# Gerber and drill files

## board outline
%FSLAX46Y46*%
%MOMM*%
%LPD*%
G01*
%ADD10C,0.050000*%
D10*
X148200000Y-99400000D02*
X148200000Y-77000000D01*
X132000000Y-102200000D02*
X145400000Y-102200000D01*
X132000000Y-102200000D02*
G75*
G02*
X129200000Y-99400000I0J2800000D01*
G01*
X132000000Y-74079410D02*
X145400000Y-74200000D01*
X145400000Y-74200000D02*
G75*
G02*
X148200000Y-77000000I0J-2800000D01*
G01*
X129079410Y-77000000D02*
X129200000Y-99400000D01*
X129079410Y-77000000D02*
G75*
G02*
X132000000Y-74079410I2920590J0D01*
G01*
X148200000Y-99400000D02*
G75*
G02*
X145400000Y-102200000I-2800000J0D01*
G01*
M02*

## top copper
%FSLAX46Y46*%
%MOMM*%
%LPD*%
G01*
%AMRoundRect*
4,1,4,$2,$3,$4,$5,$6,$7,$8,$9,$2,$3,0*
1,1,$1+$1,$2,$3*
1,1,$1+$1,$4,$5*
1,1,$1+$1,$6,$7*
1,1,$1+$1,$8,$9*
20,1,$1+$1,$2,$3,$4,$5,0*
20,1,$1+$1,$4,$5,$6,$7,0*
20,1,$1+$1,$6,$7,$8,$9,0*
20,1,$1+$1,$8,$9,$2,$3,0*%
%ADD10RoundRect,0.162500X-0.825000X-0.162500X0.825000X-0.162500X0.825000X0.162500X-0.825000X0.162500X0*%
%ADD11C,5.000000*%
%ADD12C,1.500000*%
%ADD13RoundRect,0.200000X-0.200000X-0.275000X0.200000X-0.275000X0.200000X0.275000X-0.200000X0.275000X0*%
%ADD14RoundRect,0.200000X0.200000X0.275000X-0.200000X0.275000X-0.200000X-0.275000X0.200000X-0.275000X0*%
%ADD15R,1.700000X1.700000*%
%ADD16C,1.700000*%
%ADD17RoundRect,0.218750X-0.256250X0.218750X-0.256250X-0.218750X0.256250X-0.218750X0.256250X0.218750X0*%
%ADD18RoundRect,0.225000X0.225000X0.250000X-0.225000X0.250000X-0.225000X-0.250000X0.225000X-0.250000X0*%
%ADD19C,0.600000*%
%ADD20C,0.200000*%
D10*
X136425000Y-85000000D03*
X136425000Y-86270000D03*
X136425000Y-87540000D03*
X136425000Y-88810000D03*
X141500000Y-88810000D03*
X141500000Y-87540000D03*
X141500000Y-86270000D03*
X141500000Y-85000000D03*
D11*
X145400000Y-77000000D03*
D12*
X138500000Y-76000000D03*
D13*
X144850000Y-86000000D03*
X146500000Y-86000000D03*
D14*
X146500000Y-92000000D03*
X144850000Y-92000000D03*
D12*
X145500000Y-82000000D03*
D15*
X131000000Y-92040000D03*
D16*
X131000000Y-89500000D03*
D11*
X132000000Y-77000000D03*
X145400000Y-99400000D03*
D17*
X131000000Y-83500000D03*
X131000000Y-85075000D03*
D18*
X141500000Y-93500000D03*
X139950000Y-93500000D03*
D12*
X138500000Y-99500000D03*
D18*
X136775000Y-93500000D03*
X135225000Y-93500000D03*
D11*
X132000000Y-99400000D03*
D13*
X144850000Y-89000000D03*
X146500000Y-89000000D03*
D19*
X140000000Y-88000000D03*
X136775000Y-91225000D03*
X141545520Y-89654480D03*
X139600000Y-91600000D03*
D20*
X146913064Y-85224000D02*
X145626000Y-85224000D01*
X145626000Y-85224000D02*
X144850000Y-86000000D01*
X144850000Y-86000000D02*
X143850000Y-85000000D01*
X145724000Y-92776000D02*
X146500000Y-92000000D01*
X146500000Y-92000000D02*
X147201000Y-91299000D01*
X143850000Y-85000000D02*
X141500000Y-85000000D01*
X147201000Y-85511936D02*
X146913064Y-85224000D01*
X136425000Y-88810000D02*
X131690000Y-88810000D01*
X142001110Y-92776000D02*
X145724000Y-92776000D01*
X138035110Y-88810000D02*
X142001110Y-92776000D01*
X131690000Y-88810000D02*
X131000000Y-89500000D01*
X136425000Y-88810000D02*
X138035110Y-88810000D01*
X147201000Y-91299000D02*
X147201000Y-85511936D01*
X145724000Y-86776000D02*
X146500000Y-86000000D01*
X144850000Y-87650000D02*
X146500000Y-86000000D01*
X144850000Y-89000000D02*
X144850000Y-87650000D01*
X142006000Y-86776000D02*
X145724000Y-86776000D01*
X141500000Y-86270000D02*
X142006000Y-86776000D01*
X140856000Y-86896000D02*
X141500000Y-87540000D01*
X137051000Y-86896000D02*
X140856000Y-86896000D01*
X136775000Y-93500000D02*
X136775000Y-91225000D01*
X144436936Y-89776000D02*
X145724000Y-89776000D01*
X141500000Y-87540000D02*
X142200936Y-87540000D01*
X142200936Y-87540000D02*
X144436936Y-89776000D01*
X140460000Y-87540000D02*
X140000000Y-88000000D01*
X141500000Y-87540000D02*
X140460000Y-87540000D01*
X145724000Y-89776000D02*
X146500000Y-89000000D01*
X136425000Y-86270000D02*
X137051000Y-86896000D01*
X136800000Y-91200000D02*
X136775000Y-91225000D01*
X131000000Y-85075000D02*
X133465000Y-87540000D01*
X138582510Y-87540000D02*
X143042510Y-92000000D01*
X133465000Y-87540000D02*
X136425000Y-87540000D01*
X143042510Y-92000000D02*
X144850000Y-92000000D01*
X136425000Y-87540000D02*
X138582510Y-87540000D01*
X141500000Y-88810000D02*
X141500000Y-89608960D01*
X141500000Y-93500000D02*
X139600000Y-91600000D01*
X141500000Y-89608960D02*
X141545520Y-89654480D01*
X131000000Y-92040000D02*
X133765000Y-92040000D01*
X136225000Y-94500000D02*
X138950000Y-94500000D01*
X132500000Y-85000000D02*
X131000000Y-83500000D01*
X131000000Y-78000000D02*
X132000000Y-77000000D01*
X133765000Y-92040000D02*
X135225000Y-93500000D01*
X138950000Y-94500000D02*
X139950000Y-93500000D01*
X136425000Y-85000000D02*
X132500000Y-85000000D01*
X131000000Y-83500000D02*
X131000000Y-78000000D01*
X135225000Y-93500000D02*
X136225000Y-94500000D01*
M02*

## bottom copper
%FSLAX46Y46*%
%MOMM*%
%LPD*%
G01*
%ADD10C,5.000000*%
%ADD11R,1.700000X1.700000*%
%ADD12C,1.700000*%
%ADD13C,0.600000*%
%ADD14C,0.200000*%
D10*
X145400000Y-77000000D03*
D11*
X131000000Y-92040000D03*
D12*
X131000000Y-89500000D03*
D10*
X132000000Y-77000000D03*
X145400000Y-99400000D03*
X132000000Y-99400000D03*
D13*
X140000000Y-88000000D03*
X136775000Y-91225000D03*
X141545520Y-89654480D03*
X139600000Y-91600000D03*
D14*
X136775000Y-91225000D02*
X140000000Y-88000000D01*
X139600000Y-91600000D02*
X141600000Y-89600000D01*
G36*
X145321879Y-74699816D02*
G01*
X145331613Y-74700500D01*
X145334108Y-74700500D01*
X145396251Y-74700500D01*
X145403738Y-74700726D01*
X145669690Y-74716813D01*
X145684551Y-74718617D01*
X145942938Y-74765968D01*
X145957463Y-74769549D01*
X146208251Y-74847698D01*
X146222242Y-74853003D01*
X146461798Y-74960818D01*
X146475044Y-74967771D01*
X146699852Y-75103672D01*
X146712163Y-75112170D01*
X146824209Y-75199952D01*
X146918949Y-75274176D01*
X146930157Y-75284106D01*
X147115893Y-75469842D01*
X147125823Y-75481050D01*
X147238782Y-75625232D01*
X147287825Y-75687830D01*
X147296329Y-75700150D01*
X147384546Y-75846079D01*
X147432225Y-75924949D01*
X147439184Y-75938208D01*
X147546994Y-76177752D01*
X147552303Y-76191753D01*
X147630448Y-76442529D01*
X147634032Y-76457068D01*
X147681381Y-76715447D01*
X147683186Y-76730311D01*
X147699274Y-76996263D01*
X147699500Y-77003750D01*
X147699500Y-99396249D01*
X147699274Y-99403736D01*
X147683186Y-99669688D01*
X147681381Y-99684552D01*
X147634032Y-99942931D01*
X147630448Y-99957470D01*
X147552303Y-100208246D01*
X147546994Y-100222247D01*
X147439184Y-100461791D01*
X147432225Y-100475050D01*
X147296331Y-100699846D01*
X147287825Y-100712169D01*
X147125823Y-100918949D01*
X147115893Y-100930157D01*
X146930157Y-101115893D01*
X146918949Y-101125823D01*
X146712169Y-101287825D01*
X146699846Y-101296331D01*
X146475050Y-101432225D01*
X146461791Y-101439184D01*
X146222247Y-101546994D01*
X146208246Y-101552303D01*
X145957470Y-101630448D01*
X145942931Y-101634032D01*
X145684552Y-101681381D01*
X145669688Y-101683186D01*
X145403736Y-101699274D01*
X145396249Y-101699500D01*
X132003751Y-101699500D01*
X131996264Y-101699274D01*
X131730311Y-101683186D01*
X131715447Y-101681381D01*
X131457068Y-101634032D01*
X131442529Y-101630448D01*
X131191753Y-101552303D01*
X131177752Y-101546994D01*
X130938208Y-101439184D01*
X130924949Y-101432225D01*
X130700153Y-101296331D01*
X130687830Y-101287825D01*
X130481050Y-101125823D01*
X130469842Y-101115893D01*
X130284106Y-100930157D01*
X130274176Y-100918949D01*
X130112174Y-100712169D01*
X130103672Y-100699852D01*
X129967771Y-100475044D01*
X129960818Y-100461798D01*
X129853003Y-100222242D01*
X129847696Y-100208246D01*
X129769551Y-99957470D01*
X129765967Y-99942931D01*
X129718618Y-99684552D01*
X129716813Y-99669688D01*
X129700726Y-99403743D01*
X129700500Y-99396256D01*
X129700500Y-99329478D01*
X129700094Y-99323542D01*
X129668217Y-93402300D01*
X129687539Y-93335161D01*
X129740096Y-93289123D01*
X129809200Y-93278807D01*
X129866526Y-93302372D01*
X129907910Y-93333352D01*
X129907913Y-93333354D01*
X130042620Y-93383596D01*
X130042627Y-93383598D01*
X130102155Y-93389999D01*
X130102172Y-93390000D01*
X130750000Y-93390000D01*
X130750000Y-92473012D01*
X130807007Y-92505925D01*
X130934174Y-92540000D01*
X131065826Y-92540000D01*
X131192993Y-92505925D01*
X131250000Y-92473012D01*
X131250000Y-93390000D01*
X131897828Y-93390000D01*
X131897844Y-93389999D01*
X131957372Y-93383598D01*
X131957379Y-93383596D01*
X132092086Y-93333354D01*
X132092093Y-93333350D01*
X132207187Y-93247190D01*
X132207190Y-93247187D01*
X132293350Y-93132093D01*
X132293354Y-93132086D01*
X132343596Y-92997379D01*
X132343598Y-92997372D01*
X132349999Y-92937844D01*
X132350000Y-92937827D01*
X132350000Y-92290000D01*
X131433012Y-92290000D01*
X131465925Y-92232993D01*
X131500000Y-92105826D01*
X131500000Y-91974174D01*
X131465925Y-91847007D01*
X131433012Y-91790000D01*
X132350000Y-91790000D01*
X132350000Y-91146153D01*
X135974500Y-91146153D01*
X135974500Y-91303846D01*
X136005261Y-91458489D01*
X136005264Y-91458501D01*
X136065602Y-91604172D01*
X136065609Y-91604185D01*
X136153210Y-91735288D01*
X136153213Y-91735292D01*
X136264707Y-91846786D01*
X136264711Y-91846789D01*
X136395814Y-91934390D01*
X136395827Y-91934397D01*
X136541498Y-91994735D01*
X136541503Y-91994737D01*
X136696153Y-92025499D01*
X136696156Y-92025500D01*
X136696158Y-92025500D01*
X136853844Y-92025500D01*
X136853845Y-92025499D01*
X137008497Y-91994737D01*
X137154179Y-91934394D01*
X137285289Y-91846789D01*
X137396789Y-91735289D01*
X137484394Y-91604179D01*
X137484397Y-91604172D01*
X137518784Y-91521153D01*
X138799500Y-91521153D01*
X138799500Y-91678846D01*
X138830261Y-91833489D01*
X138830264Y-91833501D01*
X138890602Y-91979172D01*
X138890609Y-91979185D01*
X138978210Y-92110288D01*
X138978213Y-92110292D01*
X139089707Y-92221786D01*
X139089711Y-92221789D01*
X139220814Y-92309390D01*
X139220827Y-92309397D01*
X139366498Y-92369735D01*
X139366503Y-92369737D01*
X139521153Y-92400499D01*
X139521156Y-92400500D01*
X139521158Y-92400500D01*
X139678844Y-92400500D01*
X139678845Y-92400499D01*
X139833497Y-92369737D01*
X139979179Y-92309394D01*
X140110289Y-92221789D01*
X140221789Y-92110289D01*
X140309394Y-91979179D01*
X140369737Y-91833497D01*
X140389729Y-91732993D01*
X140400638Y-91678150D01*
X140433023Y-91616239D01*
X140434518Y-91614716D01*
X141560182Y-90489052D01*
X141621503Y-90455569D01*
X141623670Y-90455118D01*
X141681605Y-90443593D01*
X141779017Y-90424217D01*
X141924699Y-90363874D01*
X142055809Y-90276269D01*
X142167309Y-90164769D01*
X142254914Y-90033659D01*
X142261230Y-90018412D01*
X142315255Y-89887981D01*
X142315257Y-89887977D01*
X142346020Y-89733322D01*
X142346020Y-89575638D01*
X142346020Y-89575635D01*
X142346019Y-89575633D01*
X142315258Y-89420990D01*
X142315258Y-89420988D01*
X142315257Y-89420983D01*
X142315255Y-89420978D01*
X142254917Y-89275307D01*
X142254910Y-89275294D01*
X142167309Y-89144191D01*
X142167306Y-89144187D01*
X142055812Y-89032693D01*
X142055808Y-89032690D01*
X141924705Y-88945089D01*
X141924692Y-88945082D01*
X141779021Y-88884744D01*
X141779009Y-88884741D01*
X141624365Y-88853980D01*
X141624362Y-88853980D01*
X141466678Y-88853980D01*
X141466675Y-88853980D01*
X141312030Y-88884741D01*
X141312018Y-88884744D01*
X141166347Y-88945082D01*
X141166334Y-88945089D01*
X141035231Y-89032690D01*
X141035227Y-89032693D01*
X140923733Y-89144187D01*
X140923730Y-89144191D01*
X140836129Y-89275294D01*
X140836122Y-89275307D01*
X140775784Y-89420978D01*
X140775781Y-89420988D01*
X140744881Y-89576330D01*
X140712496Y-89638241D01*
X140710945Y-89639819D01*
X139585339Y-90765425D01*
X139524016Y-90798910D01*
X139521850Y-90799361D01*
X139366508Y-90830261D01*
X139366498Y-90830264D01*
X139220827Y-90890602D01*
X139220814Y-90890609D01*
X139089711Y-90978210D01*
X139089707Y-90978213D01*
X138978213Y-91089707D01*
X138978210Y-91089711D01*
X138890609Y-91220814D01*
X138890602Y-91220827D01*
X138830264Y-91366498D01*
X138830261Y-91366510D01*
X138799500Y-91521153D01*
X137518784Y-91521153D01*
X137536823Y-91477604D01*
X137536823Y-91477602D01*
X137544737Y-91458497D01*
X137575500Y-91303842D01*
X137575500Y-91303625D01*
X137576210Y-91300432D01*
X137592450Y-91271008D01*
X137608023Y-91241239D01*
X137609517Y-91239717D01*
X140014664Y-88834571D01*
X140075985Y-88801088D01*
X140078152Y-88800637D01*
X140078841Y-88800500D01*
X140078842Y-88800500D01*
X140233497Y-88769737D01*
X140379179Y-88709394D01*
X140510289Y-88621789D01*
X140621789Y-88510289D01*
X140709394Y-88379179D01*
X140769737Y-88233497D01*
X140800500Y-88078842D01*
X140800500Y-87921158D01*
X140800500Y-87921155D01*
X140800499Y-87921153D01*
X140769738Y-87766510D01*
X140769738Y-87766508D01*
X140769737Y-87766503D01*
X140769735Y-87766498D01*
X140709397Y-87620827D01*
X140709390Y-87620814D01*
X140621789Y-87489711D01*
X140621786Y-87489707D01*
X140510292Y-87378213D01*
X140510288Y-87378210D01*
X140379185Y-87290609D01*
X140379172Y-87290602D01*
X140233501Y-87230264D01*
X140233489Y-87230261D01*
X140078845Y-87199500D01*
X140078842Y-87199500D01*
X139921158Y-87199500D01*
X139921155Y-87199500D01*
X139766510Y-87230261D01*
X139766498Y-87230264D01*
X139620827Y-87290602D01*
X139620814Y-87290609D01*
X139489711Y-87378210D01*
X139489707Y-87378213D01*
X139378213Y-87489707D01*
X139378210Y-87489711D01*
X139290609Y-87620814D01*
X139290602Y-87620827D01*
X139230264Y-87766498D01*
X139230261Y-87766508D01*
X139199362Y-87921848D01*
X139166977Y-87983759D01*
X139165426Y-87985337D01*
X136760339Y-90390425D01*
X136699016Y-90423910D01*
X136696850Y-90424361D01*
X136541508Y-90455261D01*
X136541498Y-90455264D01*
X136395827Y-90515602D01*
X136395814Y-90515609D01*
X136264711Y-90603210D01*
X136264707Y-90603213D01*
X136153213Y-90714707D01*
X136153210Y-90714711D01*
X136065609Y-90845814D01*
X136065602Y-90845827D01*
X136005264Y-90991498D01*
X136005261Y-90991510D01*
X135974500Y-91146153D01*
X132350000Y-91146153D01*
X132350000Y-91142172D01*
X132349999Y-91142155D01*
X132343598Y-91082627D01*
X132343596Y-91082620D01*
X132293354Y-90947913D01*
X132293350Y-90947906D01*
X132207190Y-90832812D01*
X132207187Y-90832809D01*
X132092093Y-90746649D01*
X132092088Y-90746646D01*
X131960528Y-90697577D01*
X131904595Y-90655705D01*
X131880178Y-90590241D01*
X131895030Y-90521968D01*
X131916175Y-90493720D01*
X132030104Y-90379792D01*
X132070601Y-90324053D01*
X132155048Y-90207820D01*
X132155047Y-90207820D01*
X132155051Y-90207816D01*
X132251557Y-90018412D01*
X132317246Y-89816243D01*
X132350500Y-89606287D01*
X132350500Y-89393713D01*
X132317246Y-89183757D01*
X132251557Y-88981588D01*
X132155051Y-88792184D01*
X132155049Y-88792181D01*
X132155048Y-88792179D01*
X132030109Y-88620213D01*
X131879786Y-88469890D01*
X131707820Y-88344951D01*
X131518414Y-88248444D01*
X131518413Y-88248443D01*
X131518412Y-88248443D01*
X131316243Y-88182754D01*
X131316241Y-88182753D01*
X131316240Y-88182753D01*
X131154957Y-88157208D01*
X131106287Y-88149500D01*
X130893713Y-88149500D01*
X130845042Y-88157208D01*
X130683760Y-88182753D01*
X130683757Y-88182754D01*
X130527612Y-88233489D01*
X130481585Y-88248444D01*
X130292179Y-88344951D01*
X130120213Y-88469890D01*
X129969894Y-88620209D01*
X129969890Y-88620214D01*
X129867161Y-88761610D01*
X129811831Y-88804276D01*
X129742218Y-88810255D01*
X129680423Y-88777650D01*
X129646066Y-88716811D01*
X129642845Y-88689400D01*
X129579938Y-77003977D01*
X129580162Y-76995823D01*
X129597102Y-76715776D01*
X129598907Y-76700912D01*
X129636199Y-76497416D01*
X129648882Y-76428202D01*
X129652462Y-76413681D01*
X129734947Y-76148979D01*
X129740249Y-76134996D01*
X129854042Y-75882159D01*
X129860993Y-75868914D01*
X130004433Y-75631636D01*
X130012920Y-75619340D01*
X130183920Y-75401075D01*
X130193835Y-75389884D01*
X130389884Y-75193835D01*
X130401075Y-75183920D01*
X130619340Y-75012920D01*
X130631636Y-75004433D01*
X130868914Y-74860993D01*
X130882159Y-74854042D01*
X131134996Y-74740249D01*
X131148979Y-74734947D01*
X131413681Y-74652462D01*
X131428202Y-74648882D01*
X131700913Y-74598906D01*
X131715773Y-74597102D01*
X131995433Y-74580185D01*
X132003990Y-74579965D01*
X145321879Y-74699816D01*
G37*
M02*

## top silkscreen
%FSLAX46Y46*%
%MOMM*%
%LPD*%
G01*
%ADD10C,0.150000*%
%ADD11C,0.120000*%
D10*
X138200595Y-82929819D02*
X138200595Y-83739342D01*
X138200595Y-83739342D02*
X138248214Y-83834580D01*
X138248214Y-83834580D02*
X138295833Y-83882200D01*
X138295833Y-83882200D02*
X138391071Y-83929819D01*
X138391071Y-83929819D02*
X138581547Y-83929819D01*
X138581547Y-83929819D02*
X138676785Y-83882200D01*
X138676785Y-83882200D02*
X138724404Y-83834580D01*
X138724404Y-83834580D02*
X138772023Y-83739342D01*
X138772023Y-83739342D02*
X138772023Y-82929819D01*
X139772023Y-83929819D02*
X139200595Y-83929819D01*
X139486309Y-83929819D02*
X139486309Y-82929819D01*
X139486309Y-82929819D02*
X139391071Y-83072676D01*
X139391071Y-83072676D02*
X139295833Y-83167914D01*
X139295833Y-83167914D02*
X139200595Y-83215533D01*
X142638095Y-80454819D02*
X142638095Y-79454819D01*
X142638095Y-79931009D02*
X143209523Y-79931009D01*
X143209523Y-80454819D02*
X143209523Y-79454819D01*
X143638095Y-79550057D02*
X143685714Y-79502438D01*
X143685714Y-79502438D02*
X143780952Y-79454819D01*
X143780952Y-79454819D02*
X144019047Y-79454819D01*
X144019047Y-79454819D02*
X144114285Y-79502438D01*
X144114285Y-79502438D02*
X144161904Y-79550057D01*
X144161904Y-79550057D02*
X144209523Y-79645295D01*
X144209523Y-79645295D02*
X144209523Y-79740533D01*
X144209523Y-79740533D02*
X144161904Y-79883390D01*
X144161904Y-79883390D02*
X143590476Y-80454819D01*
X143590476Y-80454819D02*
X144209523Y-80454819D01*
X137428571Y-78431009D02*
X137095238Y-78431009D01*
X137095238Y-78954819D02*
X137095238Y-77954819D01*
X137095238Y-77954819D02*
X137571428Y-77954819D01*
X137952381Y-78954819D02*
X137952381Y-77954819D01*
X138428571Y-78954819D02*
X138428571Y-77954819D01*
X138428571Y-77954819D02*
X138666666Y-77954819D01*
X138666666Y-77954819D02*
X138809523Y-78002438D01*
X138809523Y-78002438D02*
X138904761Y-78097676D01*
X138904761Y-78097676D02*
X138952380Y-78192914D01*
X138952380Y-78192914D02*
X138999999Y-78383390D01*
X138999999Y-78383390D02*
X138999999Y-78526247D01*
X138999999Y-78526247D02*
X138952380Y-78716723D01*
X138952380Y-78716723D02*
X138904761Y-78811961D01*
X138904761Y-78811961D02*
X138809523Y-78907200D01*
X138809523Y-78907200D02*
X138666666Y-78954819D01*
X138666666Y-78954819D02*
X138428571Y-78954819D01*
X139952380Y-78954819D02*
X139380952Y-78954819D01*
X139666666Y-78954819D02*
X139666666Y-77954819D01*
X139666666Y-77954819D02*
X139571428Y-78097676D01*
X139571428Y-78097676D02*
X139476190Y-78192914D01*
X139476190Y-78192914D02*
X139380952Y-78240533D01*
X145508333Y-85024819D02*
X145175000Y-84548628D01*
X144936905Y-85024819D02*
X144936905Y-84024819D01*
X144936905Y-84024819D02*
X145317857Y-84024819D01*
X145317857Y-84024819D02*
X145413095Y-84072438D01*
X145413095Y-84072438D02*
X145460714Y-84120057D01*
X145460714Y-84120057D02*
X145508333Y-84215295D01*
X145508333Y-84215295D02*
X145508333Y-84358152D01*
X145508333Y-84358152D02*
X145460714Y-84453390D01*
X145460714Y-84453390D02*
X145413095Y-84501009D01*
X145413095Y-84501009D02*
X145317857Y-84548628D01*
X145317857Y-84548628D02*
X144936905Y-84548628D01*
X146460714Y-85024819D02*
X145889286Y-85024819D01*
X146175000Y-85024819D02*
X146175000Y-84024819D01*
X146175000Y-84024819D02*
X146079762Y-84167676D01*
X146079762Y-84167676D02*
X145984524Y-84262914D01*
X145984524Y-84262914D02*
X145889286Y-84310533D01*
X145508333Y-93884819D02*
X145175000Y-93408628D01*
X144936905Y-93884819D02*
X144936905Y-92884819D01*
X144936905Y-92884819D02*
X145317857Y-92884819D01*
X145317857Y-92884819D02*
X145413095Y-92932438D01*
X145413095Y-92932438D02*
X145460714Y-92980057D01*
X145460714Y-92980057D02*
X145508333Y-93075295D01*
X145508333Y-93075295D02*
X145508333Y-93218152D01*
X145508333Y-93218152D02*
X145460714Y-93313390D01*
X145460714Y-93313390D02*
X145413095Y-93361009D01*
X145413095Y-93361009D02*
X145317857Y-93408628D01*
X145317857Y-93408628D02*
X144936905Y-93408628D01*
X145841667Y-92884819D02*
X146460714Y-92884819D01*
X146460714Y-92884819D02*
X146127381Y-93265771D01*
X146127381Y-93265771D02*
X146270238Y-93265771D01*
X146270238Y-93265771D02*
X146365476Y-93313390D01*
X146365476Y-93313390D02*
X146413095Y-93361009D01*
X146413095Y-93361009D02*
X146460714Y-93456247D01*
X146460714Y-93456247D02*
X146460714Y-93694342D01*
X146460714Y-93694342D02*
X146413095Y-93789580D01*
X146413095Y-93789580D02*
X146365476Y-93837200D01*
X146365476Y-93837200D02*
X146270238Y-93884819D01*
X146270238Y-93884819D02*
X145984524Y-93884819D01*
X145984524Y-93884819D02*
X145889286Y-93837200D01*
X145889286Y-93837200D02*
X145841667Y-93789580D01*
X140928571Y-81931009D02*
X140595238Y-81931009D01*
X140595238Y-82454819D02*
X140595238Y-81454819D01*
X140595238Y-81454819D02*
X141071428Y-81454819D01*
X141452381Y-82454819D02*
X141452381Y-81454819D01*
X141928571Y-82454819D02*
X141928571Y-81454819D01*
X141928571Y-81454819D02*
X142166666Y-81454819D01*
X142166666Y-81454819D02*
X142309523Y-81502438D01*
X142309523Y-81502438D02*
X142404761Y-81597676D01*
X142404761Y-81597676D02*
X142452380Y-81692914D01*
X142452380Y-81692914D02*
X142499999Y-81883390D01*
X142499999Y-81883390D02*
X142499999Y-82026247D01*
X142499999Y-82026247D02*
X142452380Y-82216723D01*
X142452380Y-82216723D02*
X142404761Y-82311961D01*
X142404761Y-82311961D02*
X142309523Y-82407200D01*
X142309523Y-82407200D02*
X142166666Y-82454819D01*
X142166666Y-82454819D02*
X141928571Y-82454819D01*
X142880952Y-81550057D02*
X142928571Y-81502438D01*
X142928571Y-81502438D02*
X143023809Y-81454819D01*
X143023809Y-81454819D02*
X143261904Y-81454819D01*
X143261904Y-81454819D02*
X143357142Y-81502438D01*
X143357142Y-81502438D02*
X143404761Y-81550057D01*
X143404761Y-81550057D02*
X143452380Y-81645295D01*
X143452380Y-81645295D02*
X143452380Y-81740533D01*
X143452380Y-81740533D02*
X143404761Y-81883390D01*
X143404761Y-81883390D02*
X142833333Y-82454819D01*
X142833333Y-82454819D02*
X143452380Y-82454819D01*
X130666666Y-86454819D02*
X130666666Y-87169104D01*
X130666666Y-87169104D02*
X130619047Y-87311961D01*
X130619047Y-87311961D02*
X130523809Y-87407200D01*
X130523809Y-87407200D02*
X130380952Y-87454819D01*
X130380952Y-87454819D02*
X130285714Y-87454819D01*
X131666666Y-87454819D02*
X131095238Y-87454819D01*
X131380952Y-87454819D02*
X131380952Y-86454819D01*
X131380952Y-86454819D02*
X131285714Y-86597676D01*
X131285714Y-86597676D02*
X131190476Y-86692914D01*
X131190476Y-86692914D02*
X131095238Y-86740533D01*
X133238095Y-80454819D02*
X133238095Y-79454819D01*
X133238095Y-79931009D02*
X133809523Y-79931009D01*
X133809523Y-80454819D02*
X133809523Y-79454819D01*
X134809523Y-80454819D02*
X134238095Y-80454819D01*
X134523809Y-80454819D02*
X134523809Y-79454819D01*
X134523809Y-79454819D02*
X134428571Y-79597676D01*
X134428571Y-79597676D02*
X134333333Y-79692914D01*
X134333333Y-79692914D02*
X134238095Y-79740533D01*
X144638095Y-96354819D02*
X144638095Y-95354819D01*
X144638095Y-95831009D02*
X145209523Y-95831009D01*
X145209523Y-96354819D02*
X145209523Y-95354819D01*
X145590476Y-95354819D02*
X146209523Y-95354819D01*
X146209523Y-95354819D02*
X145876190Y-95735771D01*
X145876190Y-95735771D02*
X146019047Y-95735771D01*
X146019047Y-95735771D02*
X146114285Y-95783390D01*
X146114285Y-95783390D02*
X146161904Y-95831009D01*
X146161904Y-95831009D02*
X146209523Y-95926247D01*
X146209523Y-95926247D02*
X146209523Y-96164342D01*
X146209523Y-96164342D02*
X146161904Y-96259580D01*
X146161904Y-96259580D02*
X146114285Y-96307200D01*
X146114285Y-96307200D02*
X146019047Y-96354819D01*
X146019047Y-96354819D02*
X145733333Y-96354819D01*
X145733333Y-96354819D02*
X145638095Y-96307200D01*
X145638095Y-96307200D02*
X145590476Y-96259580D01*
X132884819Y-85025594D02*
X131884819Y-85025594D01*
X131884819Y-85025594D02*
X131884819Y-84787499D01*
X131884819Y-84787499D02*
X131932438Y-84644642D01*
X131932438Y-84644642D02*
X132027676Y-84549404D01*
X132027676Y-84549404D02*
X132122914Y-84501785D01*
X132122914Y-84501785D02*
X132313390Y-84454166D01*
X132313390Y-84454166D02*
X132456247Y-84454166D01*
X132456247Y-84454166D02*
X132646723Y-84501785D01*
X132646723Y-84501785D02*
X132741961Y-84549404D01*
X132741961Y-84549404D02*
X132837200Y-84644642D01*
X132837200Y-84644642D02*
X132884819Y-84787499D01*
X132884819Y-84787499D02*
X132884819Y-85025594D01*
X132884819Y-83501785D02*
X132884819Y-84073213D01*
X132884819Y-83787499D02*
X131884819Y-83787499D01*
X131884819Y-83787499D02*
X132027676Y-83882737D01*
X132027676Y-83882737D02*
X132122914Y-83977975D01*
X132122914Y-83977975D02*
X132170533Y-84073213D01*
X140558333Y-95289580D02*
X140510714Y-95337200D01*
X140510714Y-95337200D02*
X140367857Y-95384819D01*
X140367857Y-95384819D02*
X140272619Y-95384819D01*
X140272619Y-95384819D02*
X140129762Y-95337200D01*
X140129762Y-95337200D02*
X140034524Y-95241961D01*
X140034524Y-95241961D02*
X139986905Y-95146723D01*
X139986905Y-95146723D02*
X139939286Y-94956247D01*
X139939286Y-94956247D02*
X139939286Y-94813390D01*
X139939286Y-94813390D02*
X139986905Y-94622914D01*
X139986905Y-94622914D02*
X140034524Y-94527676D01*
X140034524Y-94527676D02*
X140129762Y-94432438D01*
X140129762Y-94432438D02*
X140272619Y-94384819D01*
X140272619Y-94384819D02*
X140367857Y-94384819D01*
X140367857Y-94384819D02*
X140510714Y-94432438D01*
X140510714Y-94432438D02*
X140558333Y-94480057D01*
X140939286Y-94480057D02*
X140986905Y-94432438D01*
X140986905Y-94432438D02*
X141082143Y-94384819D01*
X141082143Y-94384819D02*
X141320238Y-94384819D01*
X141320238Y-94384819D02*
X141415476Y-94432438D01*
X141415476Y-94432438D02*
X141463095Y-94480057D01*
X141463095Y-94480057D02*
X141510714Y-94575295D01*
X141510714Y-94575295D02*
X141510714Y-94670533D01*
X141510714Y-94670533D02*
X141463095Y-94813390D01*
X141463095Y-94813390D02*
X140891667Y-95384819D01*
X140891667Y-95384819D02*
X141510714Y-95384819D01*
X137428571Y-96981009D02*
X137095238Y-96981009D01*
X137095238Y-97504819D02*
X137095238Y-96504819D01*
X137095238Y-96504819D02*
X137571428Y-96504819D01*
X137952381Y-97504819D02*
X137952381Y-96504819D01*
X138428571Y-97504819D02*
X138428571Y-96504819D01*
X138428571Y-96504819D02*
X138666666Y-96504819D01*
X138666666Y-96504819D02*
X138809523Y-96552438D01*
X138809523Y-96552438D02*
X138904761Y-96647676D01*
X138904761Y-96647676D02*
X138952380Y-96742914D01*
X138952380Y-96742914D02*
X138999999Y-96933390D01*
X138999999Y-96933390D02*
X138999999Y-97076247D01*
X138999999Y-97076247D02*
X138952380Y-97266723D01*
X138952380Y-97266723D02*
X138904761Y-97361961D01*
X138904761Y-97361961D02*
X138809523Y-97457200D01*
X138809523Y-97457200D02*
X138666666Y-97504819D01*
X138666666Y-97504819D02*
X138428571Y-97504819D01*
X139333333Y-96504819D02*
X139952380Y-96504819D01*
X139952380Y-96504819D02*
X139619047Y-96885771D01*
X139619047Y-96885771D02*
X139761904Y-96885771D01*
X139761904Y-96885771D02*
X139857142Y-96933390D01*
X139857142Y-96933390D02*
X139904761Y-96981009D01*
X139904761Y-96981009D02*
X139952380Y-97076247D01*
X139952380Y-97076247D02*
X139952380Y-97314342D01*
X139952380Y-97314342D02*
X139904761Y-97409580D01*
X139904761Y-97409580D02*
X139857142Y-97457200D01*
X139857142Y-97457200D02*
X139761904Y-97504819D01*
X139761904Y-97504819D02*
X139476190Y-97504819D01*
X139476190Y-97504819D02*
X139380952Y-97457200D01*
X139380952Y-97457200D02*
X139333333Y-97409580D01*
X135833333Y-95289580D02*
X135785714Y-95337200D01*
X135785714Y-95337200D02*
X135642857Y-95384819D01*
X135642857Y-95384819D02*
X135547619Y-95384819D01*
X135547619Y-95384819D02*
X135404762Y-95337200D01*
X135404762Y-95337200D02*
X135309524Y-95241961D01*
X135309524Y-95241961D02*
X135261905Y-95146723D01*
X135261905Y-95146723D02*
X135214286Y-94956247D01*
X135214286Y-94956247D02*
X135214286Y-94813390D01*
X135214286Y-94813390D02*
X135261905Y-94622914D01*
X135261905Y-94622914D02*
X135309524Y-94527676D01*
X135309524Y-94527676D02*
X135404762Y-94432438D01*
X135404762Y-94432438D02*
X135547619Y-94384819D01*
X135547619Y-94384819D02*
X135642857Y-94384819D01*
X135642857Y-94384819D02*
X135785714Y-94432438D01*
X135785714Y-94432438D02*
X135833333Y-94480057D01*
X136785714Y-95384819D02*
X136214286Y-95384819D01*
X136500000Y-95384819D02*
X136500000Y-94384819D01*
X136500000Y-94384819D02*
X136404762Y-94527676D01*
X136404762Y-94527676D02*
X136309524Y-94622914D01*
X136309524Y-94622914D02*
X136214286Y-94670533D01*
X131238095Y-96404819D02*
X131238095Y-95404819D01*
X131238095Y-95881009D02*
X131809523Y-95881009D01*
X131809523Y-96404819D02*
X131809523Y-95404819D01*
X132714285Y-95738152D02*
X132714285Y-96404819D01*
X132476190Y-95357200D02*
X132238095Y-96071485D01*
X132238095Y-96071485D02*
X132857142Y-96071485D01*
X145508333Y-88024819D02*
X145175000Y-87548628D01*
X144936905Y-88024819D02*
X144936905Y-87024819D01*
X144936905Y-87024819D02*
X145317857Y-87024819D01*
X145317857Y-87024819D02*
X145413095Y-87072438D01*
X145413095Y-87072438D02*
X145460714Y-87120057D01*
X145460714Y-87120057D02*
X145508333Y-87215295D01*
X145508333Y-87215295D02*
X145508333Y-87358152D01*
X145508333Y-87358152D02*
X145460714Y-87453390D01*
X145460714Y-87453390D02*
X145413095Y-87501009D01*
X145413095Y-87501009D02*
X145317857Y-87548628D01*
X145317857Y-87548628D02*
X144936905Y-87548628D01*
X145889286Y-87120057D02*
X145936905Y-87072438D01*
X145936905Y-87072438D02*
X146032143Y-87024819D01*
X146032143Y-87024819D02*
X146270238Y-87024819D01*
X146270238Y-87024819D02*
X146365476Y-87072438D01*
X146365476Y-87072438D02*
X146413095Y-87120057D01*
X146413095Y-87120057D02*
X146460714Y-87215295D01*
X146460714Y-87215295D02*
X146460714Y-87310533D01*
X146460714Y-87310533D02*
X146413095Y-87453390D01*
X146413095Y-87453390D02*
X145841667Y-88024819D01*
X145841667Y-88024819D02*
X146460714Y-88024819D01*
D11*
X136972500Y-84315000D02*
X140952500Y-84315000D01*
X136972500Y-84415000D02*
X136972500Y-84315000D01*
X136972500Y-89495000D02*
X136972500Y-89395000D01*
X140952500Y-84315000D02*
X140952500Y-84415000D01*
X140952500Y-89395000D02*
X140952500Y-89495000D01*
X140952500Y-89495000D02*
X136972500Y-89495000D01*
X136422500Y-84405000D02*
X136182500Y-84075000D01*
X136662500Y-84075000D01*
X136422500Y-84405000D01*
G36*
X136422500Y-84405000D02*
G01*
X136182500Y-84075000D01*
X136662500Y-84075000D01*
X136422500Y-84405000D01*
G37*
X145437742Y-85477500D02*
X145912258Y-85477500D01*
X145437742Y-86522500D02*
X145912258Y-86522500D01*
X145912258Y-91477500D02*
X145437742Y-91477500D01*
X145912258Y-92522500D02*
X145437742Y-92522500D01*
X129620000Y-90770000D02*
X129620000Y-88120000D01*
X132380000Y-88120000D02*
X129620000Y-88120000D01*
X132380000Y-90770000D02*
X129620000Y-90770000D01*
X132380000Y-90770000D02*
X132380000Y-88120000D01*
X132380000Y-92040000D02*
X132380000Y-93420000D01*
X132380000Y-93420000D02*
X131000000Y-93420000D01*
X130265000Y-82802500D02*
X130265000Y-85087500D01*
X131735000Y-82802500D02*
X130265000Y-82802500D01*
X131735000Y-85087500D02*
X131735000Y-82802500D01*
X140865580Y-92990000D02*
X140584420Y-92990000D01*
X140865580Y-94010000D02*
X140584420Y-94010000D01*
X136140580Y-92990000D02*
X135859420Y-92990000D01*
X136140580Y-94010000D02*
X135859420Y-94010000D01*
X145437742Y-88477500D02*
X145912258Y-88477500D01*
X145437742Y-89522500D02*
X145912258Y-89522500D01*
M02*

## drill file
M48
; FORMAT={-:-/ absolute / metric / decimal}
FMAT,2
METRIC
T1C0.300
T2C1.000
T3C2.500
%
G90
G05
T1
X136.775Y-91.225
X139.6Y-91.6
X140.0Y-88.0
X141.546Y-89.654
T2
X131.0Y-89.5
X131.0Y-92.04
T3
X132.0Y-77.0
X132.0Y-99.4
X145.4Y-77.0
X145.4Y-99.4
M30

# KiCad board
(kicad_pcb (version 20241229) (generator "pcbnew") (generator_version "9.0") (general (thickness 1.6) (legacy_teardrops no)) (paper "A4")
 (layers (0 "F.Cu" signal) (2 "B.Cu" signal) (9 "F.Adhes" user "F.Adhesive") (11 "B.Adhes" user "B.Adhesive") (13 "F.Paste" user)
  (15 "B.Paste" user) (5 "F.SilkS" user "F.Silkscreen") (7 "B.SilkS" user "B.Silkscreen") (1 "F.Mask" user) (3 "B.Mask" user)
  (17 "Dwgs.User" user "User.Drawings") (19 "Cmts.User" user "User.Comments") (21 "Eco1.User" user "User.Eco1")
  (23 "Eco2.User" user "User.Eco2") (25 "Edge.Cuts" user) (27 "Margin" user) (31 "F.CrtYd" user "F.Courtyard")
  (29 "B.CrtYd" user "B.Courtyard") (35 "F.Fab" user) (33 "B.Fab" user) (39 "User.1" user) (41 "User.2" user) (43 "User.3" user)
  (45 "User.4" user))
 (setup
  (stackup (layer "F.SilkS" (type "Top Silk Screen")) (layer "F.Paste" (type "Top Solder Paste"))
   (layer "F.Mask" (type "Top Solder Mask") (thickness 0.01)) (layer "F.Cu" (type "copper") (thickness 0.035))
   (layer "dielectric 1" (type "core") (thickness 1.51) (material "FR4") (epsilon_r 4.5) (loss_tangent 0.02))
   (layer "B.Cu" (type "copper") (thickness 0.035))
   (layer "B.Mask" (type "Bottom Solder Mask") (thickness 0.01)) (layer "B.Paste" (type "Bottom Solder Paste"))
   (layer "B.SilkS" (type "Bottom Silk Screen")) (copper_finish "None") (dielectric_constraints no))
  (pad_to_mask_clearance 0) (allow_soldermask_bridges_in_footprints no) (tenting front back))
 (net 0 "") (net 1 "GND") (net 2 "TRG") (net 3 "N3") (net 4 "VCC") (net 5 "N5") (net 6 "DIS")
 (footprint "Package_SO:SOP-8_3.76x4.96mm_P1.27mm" (layer "F.Cu") (at 138.9625 86.905)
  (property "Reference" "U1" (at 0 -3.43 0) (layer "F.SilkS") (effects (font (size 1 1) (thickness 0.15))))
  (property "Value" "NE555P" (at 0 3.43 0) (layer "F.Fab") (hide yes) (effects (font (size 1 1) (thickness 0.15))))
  (fp_line (start -1.99 -2.59) (end 1.99 -2.59) (stroke (width 0.12) (type solid)) (layer "F.SilkS"))
  (fp_line (start -1.99 -2.49) (end -1.99 -2.59) (stroke (width 0.12) (type solid)) (layer "F.SilkS"))
  (fp_line (start -1.99 2.59) (end -1.99 2.49) (stroke (width 0.12) (type solid)) (layer "F.SilkS"))
  (fp_line (start 1.99 -2.59) (end 1.99 -2.49) (stroke (width 0.12) (type solid)) (layer "F.SilkS"))
  (fp_line (start 1.99 2.49) (end 1.99 2.59) (stroke (width 0.12) (type solid)) (layer "F.SilkS"))
  (fp_line (start 1.99 2.59) (end -1.99 2.59) (stroke (width 0.12) (type solid)) (layer "F.SilkS"))
  (fp_poly (pts (xy -2.54 -2.5) (xy -2.78 -2.83) (xy -2.3 -2.83)) (stroke (width 0.12) (type solid)) (fill yes) (layer "F.SilkS"))
  (pad "1" smd roundrect (at -2.5375 -1.905) (size 1.975 0.65) (layers "F.Cu" "F.Mask" "F.Paste") (roundrect_rratio 0.25) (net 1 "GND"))
  (pad "2" smd roundrect (at -2.5375 -0.635) (size 1.975 0.65) (layers "F.Cu" "F.Mask" "F.Paste") (roundrect_rratio 0.25) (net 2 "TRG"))
  (pad "3" smd roundrect (at -2.5375 0.635) (size 1.975 0.65) (layers "F.Cu" "F.Mask" "F.Paste") (roundrect_rratio 0.25) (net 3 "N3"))
  (pad "4" smd roundrect (at -2.5375 1.905) (size 1.975 0.65) (layers "F.Cu" "F.Mask" "F.Paste") (roundrect_rratio 0.25) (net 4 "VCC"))
  (pad "5" smd roundrect (at 2.5375 1.905) (size 1.975 0.65) (layers "F.Cu" "F.Mask" "F.Paste") (roundrect_rratio 0.25) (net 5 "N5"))
  (pad "6" smd roundrect (at 2.5375 0.635) (size 1.975 0.65) (layers "F.Cu" "F.Mask" "F.Paste") (roundrect_rratio 0.25) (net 2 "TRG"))
  (pad "7" smd roundrect (at 2.5375 -0.635) (size 1.975 0.65) (layers "F.Cu" "F.Mask" "F.Paste") (roundrect_rratio 0.25) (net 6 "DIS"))
  (pad "8" smd roundrect (at 2.5375 -1.905) (size 1.975 0.65) (layers "F.Cu" "F.Mask" "F.Paste") (roundrect_rratio 0.25) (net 4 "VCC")))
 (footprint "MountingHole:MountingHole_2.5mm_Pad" (layer "F.Cu") (at 145.4 77)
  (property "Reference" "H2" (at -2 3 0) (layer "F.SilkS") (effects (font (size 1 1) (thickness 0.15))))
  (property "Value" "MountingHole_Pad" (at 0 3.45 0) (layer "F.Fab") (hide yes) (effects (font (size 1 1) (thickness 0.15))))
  (pad "1" thru_hole circle (at 0 0) (size 5 5) (drill 2.5) (layers "*.Cu" "*.Mask") (remove_unused_layers no) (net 1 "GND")
   (zone_connect 2)))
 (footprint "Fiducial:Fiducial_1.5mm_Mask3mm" (layer "F.Cu") (at 138.5 76)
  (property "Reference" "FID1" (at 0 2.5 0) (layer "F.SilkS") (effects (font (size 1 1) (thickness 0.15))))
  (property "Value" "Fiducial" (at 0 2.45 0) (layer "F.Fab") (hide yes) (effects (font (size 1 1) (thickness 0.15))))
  (pad "" smd circle (at 0 0) (size 1.5 1.5) (layers "F.Cu" "F.Mask") (solder_mask_margin 0.75) (clearance 0.85)))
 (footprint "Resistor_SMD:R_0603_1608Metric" (layer "F.Cu") (at 145.675 86)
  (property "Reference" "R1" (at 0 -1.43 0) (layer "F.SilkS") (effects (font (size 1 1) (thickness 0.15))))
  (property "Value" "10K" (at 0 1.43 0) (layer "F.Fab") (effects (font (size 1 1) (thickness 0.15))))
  (fp_line (start -0.237258 -0.5225) (end 0.237258 -0.5225) (stroke (width 0.12) (type solid)) (layer "F.SilkS"))
  (fp_line (start -0.237258 0.5225) (end 0.237258 0.5225) (stroke (width 0.12) (type solid)) (layer "F.SilkS"))
  (pad "1" smd roundrect (at -0.825 0) (size 0.8 0.95) (layers "F.Cu" "F.Mask" "F.Paste") (roundrect_rratio 0.25) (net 4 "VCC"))
  (pad "2" smd roundrect (at 0.825 0) (size 0.8 0.95) (layers "F.Cu" "F.Mask" "F.Paste") (roundrect_rratio 0.25) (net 6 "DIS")))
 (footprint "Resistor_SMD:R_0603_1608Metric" (layer "F.Cu") (at 145.675 92 180)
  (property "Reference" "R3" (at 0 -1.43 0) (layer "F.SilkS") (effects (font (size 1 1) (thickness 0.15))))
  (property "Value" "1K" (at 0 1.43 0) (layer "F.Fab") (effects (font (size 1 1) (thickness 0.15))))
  (fp_line (start -0.237258 0.5225) (end 0.237258 0.5225) (stroke (width 0.12) (type solid)) (layer "F.SilkS"))
  (fp_line (start -0.237258 -0.5225) (end 0.237258 -0.5225) (stroke (width 0.12) (type solid)) (layer "F.SilkS"))
  (pad "1" smd roundrect (at -0.825 0 180) (size 0.8 0.95) (layers "F.Cu" "F.Mask" "F.Paste") (roundrect_rratio 0.25) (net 4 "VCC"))
  (pad "2" smd roundrect (at 0.825 0 180) (size 0.8 0.95) (layers "F.Cu" "F.Mask" "F.Paste") (roundrect_rratio 0.25) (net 3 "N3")))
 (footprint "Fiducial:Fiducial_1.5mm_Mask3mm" (layer "F.Cu") (at 145.5 82)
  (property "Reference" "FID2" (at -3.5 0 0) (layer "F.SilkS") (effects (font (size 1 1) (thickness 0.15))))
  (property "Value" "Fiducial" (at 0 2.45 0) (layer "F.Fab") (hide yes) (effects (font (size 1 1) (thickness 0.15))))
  (pad "" smd circle (at 0 0) (size 1.5 1.5) (layers "F.Cu" "F.Mask") (solder_mask_margin 0.75) (clearance 0.85)))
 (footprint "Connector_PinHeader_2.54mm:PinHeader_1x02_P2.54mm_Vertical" (layer "F.Cu") (at 131 92.04 180)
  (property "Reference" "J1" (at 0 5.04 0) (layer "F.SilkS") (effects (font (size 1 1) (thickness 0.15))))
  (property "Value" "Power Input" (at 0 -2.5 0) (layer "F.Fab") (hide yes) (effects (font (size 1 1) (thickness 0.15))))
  (fp_line (start 1.38 1.27) (end 1.38 3.92) (stroke (width 0.12) (type solid)) (layer "F.SilkS"))
  (fp_line (start -1.38 3.92) (end 1.38 3.92) (stroke (width 0.12) (type solid)) (layer "F.SilkS"))
  (fp_line (start -1.38 1.27) (end 1.38 1.27) (stroke (width 0.12) (type solid)) (layer "F.SilkS"))
  (fp_line (start -1.38 1.27) (end -1.38 3.92) (stroke (width 0.12) (type solid)) (layer "F.SilkS"))
  (fp_line (start -1.38 0) (end -1.38 -1.38) (stroke (width 0.12) (type solid)) (layer "F.SilkS"))
  (fp_line (start -1.38 -1.38) (end 0 -1.38) (stroke (width 0.12) (type solid)) (layer "F.SilkS"))
  (pad "1" thru_hole rect (at 0 0 180) (size 1.7 1.7) (drill 1) (layers "*.Cu" "*.Mask") (remove_unused_layers no) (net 1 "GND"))
  (pad "2" thru_hole circle (at 0 2.54 180) (size 1.7 1.7) (drill 1) (layers "*.Cu" "*.Mask") (remove_unused_layers no) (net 4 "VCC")))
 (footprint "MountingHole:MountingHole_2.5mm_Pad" (layer "F.Cu") (at 132 77)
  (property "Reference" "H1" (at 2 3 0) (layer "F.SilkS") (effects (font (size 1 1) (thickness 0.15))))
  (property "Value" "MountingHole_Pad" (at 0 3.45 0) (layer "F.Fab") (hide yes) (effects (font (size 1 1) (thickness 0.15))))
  (pad "1" thru_hole circle (at 0 0) (size 5 5) (drill 2.5) (layers "*.Cu" "*.Mask") (remove_unused_layers no) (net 1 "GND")
   (zone_connect 2)))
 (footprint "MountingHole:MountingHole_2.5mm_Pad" (layer "F.Cu") (at 145.4 99.4)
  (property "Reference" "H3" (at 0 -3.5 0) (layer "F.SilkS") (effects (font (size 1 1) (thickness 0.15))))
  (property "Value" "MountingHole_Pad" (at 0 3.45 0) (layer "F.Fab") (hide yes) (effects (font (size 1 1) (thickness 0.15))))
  (pad "1" thru_hole circle (at 0 0) (size 5 5) (drill 2.5) (layers "*.Cu" "*.Mask") (remove_unused_layers no) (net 1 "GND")
   (zone_connect 2)))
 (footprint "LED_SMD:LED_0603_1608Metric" (layer "F.Cu") (at 131 84.2875 -90)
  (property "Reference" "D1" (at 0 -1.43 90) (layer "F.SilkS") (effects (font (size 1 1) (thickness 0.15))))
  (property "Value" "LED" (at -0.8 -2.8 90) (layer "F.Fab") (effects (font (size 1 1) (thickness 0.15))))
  (fp_line (start -1.485 0.735) (end 0.8 0.735) (stroke (width 0.12) (type solid)) (layer "F.SilkS"))
  (fp_line (start -1.485 -0.735) (end -1.485 0.735) (stroke (width 0.12) (type solid)) (layer "F.SilkS"))
  (fp_line (start 0.8 -0.735) (end -1.485 -0.735) (stroke (width 0.12) (type solid)) (layer "F.SilkS"))
  (pad "1" smd roundrect (at -0.7875 0 270) (size 0.875 0.95) (layers "F.Cu" "F.Mask" "F.Paste") (roundrect_rratio 0.25) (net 1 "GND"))
  (pad "2" smd roundrect (at 0.7875 0 270) (size 0.875 0.95) (layers "F.Cu" "F.Mask" "F.Paste") (roundrect_rratio 0.25) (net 3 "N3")))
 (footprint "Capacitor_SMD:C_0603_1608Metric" (layer "F.Cu") (at 140.725 93.5 180)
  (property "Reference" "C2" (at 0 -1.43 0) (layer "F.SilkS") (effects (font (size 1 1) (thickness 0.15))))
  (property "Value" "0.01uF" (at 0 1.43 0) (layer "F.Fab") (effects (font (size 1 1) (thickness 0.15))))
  (fp_line (start -0.14058 0.51) (end 0.14058 0.51) (stroke (width 0.12) (type solid)) (layer "F.SilkS"))
  (fp_line (start -0.14058 -0.51) (end 0.14058 -0.51) (stroke (width 0.12) (type solid)) (layer "F.SilkS"))
  (pad "1" smd roundrect (at -0.775 0 180) (size 0.9 0.95) (layers "F.Cu" "F.Mask" "F.Paste") (roundrect_rratio 0.25) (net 5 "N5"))
  (pad "2" smd roundrect (at 0.775 0 180) (size 0.9 0.95) (layers "F.Cu" "F.Mask" "F.Paste") (roundrect_rratio 0.25) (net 1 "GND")))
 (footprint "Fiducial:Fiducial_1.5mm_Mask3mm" (layer "F.Cu") (at 138.5 99.5)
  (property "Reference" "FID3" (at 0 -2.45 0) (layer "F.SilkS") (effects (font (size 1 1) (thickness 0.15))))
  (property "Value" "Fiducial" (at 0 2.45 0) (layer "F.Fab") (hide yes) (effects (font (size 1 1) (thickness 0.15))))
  (pad "" smd circle (at 0 0) (size 1.5 1.5) (layers "F.Cu" "F.Mask") (solder_mask_margin 0.75) (clearance 0.85)))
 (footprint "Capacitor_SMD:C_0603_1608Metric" (layer "F.Cu") (at 136 93.5 180)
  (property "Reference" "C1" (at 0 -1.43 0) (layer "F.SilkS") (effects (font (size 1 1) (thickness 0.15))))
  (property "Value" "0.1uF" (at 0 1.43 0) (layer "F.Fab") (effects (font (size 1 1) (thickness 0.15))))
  (fp_line (start -0.14058 0.51) (end 0.14058 0.51) (stroke (width 0.12) (type solid)) (layer "F.SilkS"))
  (fp_line (start -0.14058 -0.51) (end 0.14058 -0.51) (stroke (width 0.12) (type solid)) (layer "F.SilkS"))
  (pad "1" smd roundrect (at -0.775 0 180) (size 0.9 0.95) (layers "F.Cu" "F.Mask" "F.Paste") (roundrect_rratio 0.25) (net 2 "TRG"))
  (pad "2" smd roundrect (at 0.775 0 180) (size 0.9 0.95) (layers "F.Cu" "F.Mask" "F.Paste") (roundrect_rratio 0.25) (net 1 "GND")))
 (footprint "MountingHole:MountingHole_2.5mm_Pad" (layer "F.Cu") (at 132 99.4)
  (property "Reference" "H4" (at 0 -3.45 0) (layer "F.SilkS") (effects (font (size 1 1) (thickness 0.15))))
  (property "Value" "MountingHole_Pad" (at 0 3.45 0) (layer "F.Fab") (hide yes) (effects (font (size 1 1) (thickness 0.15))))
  (pad "1" thru_hole circle (at 0 0) (size 5 5) (drill 2.5) (layers "*.Cu" "*.Mask") (remove_unused_layers no) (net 1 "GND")
   (zone_connect 2)))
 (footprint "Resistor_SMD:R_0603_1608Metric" (layer "F.Cu") (at 145.675 89)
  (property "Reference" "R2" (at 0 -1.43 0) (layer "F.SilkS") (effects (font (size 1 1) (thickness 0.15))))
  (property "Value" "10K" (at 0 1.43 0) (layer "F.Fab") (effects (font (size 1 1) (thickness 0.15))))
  (fp_line (start -0.237258 -0.5225) (end 0.237258 -0.5225) (stroke (width 0.12) (type solid)) (layer "F.SilkS"))
  (fp_line (start -0.237258 0.5225) (end 0.237258 0.5225) (stroke (width 0.12) (type solid)) (layer "F.SilkS"))
  (pad "1" smd roundrect (at -0.825 0) (size 0.8 0.95) (layers "F.Cu" "F.Mask" "F.Paste") (roundrect_rratio 0.25) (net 6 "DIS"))
  (pad "2" smd roundrect (at 0.825 0) (size 0.8 0.95) (layers "F.Cu" "F.Mask" "F.Paste") (roundrect_rratio 0.25) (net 2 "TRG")))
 (gr_line (start 148.2 99.4) (end 148.2 77) (stroke (width 0.05) (type default)) (layer "Edge.Cuts"))
 (gr_line (start 132 102.2) (end 145.4 102.2) (stroke (width 0.05) (type default)) (layer "Edge.Cuts"))
 (gr_arc (start 132 102.2) (mid 130.020101 101.379899) (end 129.2 99.4) (stroke (width 0.05) (type default)) (layer "Edge.Cuts"))
 (gr_line (start 132 74.07941) (end 145.4 74.2) (stroke (width 0.05) (type default)) (layer "Edge.Cuts"))
 (gr_arc (start 145.4 74.2) (mid 147.379899 75.020101) (end 148.2 77) (stroke (width 0.05) (type default)) (layer "Edge.Cuts"))
 (gr_line (start 129.07941 77) (end 129.2 99.4) (stroke (width 0.05) (type default)) (layer "Edge.Cuts"))
 (gr_arc (start 129.07941 77) (mid 129.934831 74.934831) (end 132 74.07941) (stroke (width 0.05) (type default)) (layer "Edge.Cuts"))
 (gr_arc (start 148.2 99.4) (mid 147.379899 101.379899) (end 145.4 102.2) (stroke (width 0.05) (type default)) (layer "Edge.Cuts"))
 (segment (start 146.913064 85.224) (end 145.626 85.224) (width 0.2) (layer "F.Cu") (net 4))
 (segment (start 145.626 85.224) (end 144.85 86) (width 0.2) (layer "F.Cu") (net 4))
 (segment (start 144.85 86) (end 143.85 85) (width 0.2) (layer "F.Cu") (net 4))
 (segment (start 145.724 92.776) (end 146.5 92) (width 0.2) (layer "F.Cu") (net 4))
 (segment (start 146.5 92) (end 147.201 91.299) (width 0.2) (layer "F.Cu") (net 4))
 (segment (start 143.85 85) (end 141.5 85) (width 0.2) (layer "F.Cu") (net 4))
 (segment (start 147.201 85.511936) (end 146.913064 85.224) (width 0.2) (layer "F.Cu") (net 4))
 (segment (start 136.425 88.81) (end 131.69 88.81) (width 0.2) (layer "F.Cu") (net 4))
 (segment (start 142.00111 92.776) (end 145.724 92.776) (width 0.2) (layer "F.Cu") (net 4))
 (segment (start 138.03511 88.81) (end 142.00111 92.776) (width 0.2) (layer "F.Cu") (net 4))
 (segment (start 131.69 88.81) (end 131 89.5) (width 0.2) (layer "F.Cu") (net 4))
 (segment (start 136.425 88.81) (end 138.03511 88.81) (width 0.2) (layer "F.Cu") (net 4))
 (segment (start 147.201 91.299) (end 147.201 85.511936) (width 0.2) (layer "F.Cu") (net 4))
 (segment (start 145.724 86.776) (end 146.5 86) (width 0.2) (layer "F.Cu") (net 6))
 (segment (start 144.85 87.65) (end 146.5 86) (width 0.2) (layer "F.Cu") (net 6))
 (segment (start 144.85 89) (end 144.85 87.65) (width 0.2) (layer "F.Cu") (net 6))
 (segment (start 142.006 86.776) (end 145.724 86.776) (width 0.2) (layer "F.Cu") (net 6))
 (segment (start 141.5 86.27) (end 142.006 86.776) (width 0.2) (layer "F.Cu") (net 6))
 (segment (start 140.856 86.896) (end 141.5 87.54) (width 0.2) (layer "F.Cu") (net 2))
 (segment (start 137.051 86.896) (end 140.856 86.896) (width 0.2) (layer "F.Cu") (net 2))
 (segment (start 136.775 93.5) (end 136.775 91.225) (width 0.2) (layer "F.Cu") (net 2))
 (segment (start 144.436936 89.776) (end 145.724 89.776) (width 0.2) (layer "F.Cu") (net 2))
 (segment (start 141.5 87.54) (end 142.200936 87.54) (width 0.2) (layer "F.Cu") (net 2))
 (segment (start 142.200936 87.54) (end 144.436936 89.776) (width 0.2) (layer "F.Cu") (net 2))
 (segment (start 140.46 87.54) (end 140 88) (width 0.2) (layer "F.Cu") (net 2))
 (segment (start 141.5 87.54) (end 140.46 87.54) (width 0.2) (layer "F.Cu") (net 2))
 (segment (start 145.724 89.776) (end 146.5 89) (width 0.2) (layer "F.Cu") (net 2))
 (segment (start 136.425 86.27) (end 137.051 86.896) (width 0.2) (layer "F.Cu") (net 2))
 (segment (start 136.8 91.2) (end 136.775 91.225) (width 0.2) (layer "F.Cu") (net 2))
 (via (at 140 88) (size 0.6) (drill 0.3) (layers "F.Cu" "B.Cu") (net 2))
 (via (at 136.775 91.225) (size 0.6) (drill 0.3) (layers "F.Cu" "B.Cu") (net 2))
 (segment (start 136.775 91.225) (end 140 88) (width 0.2) (layer "B.Cu") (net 2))
 (segment (start 131 85.075) (end 133.465 87.54) (width 0.2) (layer "F.Cu") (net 3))
 (segment (start 138.58251 87.54) (end 143.04251 92) (width 0.2) (layer "F.Cu") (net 3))
 (segment (start 133.465 87.54) (end 136.425 87.54) (width 0.2) (layer "F.Cu") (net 3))
 (segment (start 143.04251 92) (end 144.85 92) (width 0.2) (layer "F.Cu") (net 3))
 (segment (start 136.425 87.54) (end 138.58251 87.54) (width 0.2) (layer "F.Cu") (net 3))
 (segment (start 141.5 88.81) (end 141.5 89.60896) (width 0.2) (layer "F.Cu") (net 5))
 (segment (start 141.5 93.5) (end 139.6 91.6) (width 0.2) (layer "F.Cu") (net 5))
 (segment (start 141.5 89.60896) (end 141.54552 89.65448) (width 0.2) (layer "F.Cu") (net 5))
 (via (at 141.54552 89.65448) (size 0.6) (drill 0.3) (layers "F.Cu" "B.Cu") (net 5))
 (via (at 139.6 91.6) (size 0.6) (drill 0.3) (layers "F.Cu" "B.Cu") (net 5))
 (segment (start 139.6 91.6) (end 141.6 89.6) (width 0.2) (layer "B.Cu") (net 5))
 (segment (start 131 92.04) (end 133.765 92.04) (width 0.2) (layer "F.Cu") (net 1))
 (segment (start 136.225 94.5) (end 138.95 94.5) (width 0.2) (layer "F.Cu") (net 1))
 (segment (start 132.5 85) (end 131 83.5) (width 0.2) (layer "F.Cu") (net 1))
 (segment (start 131 78) (end 132 77) (width 0.2) (layer "F.Cu") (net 1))
 (segment (start 133.765 92.04) (end 135.225 93.5) (width 0.2) (layer "F.Cu") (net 1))
 (segment (start 138.95 94.5) (end 139.95 93.5) (width 0.2) (layer "F.Cu") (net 1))
 (segment (start 136.425 85) (end 132.5 85) (width 0.2) (layer "F.Cu") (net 1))
 (segment (start 131 83.5) (end 131 78) (width 0.2) (layer "F.Cu") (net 1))
 (segment (start 135.225 93.5) (end 136.225 94.5) (width 0.2) (layer "F.Cu") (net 1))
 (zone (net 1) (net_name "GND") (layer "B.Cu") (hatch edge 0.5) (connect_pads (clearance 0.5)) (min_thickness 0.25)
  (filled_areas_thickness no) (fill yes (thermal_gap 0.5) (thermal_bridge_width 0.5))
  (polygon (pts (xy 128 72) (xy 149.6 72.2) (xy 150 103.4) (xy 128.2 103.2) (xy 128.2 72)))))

